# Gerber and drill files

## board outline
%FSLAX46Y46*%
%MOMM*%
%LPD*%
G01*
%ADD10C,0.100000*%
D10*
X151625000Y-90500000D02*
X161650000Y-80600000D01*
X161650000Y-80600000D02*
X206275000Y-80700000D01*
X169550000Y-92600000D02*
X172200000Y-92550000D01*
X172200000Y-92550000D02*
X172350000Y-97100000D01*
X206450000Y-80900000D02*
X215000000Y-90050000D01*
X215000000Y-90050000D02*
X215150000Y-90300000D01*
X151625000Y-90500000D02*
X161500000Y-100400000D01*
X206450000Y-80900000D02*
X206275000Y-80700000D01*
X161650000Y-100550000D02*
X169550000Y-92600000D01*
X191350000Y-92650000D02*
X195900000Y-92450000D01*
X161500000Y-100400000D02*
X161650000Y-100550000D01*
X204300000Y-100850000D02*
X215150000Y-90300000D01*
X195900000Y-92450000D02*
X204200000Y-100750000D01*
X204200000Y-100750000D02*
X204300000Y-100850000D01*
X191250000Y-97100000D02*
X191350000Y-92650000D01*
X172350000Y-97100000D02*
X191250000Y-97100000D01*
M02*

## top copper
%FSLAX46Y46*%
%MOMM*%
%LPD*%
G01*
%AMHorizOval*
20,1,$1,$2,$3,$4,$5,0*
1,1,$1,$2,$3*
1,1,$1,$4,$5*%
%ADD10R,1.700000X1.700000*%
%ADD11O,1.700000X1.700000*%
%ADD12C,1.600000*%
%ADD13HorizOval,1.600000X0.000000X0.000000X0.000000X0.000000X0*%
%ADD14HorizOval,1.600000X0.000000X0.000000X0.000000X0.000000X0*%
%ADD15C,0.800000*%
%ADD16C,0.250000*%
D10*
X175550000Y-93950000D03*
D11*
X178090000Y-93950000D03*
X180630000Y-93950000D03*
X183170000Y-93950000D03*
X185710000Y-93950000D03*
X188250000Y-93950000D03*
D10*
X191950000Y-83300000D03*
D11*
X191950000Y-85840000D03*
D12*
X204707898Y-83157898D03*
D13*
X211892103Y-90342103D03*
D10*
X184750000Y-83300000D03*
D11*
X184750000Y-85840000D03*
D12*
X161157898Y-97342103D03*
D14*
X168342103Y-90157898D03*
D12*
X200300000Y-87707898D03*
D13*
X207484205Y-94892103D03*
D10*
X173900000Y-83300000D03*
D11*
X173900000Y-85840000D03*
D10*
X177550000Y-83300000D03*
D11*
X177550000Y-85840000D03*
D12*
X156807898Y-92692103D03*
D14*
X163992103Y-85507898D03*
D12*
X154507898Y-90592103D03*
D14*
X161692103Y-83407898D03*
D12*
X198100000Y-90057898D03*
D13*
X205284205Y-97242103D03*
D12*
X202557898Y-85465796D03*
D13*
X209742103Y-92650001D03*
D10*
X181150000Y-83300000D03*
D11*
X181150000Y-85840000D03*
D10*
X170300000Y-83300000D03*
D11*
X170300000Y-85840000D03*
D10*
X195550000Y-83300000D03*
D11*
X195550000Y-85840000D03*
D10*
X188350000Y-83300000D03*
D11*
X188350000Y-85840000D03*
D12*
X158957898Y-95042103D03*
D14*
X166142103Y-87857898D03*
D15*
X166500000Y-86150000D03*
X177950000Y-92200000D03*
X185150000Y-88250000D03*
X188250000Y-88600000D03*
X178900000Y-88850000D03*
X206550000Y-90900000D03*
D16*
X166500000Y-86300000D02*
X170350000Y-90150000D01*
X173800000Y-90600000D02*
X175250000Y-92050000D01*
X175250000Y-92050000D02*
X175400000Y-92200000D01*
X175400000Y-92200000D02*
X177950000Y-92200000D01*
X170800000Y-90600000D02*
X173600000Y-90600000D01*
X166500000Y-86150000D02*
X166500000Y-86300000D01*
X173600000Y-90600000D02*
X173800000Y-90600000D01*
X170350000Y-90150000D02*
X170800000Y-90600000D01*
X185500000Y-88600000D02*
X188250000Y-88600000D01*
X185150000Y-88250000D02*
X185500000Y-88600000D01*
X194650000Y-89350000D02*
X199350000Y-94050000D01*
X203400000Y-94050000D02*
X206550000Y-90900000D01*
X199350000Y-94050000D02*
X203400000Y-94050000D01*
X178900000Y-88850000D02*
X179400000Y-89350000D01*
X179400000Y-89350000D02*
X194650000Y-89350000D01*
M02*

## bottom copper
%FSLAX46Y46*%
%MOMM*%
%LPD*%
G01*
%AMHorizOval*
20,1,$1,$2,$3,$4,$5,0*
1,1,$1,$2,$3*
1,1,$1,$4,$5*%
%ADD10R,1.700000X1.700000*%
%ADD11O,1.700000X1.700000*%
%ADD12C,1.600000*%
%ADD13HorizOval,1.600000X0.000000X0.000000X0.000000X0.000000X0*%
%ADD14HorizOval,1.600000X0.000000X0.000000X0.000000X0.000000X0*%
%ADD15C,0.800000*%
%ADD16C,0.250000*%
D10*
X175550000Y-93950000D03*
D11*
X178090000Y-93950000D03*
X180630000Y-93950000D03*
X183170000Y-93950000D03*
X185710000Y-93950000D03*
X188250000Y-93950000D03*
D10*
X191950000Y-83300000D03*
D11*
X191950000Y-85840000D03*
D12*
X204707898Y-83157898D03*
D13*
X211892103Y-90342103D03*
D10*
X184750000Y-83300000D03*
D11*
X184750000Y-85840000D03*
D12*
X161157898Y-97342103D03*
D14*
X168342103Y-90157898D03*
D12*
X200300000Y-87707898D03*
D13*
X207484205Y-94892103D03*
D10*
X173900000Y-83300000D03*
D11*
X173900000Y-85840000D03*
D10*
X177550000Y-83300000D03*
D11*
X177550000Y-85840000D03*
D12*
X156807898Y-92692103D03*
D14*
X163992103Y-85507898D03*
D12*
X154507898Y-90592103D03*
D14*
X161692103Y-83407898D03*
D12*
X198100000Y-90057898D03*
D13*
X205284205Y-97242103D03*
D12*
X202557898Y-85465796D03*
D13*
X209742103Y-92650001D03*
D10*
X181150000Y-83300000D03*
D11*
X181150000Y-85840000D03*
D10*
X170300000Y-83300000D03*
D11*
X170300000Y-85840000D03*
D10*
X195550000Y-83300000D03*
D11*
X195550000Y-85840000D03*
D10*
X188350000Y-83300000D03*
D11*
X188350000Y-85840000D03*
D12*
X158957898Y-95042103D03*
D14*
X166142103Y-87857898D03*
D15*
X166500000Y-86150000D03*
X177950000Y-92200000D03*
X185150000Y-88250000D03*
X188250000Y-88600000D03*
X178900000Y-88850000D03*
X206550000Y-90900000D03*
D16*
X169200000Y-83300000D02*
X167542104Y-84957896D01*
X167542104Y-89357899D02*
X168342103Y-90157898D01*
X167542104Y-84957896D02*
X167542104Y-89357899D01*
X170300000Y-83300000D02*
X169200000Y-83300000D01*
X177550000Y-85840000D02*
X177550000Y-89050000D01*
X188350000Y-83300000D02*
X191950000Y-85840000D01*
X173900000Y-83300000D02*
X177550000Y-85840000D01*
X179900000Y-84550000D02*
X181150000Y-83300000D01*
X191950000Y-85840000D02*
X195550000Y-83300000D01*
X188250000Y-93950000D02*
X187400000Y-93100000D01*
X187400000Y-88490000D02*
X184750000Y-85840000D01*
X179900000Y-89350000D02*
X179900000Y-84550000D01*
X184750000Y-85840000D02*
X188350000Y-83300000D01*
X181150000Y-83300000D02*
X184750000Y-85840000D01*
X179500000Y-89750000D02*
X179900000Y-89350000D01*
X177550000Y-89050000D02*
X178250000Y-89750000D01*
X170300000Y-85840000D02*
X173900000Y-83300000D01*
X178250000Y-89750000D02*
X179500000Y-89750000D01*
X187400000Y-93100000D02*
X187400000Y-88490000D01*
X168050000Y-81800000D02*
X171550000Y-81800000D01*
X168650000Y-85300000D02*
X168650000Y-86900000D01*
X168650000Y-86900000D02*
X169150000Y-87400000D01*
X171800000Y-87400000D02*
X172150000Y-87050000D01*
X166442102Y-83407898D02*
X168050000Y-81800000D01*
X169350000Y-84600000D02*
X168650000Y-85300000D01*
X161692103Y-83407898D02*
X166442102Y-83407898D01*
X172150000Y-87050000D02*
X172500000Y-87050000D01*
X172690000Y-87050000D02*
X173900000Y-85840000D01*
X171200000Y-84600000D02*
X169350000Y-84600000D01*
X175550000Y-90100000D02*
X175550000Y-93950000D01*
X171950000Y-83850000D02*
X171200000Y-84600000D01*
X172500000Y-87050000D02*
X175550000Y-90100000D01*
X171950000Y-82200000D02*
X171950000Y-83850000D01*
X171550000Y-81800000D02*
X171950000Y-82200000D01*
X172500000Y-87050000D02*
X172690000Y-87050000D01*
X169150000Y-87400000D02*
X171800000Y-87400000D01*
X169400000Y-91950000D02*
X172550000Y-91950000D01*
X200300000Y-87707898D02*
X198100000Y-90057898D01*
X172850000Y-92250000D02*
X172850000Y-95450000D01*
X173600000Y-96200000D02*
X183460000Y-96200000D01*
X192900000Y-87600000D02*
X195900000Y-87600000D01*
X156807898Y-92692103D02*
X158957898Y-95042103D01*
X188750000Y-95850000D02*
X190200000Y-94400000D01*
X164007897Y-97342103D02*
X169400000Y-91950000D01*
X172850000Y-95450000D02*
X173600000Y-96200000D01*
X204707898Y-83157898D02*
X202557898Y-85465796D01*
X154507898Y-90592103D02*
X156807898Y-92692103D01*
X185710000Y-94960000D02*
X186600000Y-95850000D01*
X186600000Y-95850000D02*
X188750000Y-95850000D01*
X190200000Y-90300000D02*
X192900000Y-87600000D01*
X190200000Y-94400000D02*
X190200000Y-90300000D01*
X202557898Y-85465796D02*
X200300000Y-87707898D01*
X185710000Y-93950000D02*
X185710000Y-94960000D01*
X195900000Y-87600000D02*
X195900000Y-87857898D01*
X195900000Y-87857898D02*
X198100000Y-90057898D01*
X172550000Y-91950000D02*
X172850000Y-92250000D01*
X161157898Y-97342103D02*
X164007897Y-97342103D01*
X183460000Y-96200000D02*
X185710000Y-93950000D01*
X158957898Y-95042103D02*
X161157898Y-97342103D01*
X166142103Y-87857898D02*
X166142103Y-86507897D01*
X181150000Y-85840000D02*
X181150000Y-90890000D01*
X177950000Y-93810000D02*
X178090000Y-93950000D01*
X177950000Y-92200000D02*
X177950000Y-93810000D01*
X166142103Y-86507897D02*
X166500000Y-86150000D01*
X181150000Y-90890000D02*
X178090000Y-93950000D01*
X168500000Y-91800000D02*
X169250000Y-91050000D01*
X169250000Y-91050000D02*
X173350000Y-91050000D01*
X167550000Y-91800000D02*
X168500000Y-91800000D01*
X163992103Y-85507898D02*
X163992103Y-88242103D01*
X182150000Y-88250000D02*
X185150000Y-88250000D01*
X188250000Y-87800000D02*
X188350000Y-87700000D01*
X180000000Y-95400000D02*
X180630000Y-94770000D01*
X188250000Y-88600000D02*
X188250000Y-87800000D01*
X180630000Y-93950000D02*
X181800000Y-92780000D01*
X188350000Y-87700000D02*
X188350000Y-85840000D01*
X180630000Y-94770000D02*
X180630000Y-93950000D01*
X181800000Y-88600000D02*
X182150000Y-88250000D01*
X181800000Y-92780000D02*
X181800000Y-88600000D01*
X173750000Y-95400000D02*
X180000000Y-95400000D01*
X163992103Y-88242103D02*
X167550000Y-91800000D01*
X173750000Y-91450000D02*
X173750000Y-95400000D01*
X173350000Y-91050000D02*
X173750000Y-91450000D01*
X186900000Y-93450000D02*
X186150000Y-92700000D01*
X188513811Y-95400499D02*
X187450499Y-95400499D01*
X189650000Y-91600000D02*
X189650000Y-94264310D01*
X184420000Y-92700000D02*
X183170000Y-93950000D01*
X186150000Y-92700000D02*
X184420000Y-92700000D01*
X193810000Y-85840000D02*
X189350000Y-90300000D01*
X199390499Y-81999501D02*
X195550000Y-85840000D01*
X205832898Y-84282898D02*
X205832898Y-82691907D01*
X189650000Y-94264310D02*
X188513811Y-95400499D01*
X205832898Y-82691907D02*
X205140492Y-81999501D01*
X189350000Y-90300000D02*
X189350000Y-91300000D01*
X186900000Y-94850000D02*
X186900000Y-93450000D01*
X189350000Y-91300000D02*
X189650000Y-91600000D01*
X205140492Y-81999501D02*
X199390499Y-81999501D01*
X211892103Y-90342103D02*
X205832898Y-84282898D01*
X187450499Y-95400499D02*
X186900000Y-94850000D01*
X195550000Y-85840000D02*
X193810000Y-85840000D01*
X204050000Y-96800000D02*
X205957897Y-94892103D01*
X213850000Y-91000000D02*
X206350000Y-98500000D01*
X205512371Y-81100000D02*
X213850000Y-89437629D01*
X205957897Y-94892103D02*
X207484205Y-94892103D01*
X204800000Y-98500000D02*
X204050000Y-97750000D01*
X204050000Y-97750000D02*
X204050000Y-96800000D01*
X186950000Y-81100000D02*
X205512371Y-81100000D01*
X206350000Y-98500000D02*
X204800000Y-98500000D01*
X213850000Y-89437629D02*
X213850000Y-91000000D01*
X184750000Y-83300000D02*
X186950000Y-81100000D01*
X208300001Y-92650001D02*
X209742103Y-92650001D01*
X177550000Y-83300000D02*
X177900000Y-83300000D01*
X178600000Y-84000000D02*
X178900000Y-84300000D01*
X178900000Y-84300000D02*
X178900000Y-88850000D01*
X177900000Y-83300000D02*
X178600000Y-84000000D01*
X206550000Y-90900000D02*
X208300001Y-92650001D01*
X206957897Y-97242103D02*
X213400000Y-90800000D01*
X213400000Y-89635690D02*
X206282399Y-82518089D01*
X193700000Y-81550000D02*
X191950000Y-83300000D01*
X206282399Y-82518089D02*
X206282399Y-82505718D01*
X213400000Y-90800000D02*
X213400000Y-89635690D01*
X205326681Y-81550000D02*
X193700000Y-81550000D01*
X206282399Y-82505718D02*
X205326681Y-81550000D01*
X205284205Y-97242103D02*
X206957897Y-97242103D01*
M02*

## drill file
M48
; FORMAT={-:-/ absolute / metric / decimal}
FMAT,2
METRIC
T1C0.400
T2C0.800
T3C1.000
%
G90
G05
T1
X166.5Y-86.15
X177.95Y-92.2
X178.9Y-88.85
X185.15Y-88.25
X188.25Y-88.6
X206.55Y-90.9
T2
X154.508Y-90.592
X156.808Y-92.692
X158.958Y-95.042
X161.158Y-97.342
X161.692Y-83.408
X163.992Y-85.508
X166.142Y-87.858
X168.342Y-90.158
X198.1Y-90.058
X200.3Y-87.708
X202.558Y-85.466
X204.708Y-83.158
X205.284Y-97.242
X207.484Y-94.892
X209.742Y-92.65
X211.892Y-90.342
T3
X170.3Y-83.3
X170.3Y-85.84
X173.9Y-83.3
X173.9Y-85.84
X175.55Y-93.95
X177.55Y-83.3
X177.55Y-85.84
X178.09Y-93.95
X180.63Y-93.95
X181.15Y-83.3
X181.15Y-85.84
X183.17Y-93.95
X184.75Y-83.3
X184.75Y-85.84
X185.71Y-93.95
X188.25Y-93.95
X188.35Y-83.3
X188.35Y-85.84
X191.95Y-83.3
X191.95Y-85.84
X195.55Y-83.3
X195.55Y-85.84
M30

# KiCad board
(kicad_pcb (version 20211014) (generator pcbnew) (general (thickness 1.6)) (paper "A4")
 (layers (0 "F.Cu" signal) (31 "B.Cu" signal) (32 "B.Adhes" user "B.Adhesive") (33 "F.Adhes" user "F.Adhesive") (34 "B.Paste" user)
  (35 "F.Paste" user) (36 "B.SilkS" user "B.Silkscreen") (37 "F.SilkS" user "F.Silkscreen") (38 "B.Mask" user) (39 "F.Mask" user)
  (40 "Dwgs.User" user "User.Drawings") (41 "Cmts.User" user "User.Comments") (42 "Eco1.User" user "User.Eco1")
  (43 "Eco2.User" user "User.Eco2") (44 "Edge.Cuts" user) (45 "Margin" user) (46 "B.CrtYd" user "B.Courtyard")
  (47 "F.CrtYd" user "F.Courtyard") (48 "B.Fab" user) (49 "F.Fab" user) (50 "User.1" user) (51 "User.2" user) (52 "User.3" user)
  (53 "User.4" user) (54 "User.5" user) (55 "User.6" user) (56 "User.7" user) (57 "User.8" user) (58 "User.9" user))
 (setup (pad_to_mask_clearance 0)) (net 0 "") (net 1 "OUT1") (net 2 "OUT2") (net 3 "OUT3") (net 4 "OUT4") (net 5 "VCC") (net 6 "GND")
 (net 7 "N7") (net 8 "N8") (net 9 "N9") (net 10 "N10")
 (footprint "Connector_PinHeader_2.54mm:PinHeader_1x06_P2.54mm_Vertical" (layer "F.Cu") (at 175.55 93.95 90)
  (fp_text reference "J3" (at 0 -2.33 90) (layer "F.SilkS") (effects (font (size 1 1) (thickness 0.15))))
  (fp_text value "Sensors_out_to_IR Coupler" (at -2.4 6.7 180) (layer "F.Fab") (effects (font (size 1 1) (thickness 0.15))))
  (pad "1" thru_hole rect (at 0 0 90) (size 1.7 1.7) (drill 1) (layers *.Cu *.Mask) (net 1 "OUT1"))
  (pad "2" thru_hole oval (at 0 2.54 90) (size 1.7 1.7) (drill 1) (layers *.Cu *.Mask) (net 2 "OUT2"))
  (pad "3" thru_hole oval (at 0 5.08 90) (size 1.7 1.7) (drill 1) (layers *.Cu *.Mask) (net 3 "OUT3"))
  (pad "4" thru_hole oval (at 0 7.62 90) (size 1.7 1.7) (drill 1) (layers *.Cu *.Mask) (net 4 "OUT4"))
  (pad "5" thru_hole oval (at 0 10.16 90) (size 1.7 1.7) (drill 1) (layers *.Cu *.Mask) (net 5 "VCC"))
  (pad "6" thru_hole oval (at 0 12.7 90) (size 1.7 1.7) (drill 1) (layers *.Cu *.Mask) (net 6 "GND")))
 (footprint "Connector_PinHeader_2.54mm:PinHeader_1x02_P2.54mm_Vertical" (layer "F.Cu") (at 191.95 83.3)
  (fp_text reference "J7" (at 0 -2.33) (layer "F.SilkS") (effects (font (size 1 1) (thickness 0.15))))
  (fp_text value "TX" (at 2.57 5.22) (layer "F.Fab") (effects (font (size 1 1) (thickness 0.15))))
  (pad "1" thru_hole rect (at 0 0) (size 1.7 1.7) (drill 1) (layers *.Cu *.Mask) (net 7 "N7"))
  (pad "2" thru_hole oval (at 0 2.54) (size 1.7 1.7) (drill 1) (layers *.Cu *.Mask) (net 6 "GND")))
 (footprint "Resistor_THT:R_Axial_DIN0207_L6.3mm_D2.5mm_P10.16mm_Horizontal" (layer "F.Cu") (at 204.707898 83.157898 -45)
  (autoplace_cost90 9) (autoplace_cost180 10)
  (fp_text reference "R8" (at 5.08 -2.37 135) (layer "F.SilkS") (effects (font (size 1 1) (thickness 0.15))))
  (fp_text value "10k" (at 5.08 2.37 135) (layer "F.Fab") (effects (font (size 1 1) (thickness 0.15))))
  (pad "1" thru_hole circle (at 0 0 315) (size 1.6 1.6) (drill 0.8) (layers *.Cu *.Mask) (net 5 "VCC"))
  (pad "2" thru_hole oval (at 10.16 0 315) (size 1.6 1.6) (drill 0.8) (layers *.Cu *.Mask) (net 4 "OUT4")))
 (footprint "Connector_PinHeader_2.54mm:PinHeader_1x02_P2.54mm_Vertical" (layer "F.Cu") (at 184.75 83.3)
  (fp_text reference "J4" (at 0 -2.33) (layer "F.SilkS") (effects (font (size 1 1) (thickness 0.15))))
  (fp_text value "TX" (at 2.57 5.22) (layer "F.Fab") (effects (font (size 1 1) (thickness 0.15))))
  (pad "1" thru_hole rect (at 0 0) (size 1.7 1.7) (drill 1) (layers *.Cu *.Mask) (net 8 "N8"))
  (pad "2" thru_hole oval (at 0 2.54) (size 1.7 1.7) (drill 1) (layers *.Cu *.Mask) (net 6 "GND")))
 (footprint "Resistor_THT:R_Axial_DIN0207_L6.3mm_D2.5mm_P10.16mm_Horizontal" (layer "F.Cu") (at 161.157898 97.342103 45)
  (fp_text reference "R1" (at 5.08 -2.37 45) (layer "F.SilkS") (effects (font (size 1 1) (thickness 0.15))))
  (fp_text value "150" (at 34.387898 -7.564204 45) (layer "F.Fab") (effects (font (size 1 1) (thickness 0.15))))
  (pad "1" thru_hole circle (at 0 0 45) (size 1.6 1.6) (drill 0.8) (layers *.Cu *.Mask) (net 5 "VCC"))
  (pad "2" thru_hole oval (at 10.16 0 45) (size 1.6 1.6) (drill 0.8) (layers *.Cu *.Mask) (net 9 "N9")))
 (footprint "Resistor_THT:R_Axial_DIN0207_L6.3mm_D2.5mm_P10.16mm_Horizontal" (layer "F.Cu") (at 200.3 87.707898 -45)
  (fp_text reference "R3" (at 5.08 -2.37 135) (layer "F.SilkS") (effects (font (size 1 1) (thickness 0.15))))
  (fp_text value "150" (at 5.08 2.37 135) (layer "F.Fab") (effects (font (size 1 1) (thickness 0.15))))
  (pad "1" thru_hole circle (at 0 0 315) (size 1.6 1.6) (drill 0.8) (layers *.Cu *.Mask) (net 5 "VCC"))
  (pad "2" thru_hole oval (at 10.16 0 315) (size 1.6 1.6) (drill 0.8) (layers *.Cu *.Mask) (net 8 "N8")))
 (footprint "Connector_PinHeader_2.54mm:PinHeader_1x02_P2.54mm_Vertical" (layer "F.Cu") (at 173.9 83.3)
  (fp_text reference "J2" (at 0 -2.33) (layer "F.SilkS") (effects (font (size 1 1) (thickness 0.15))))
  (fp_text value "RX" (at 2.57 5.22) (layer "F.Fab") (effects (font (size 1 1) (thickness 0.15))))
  (pad "1" thru_hole rect (at 0 0) (size 1.7 1.7) (drill 1) (layers *.Cu *.Mask) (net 6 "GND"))
  (pad "2" thru_hole oval (at 0 2.54) (size 1.7 1.7) (drill 1) (layers *.Cu *.Mask) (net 1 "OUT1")))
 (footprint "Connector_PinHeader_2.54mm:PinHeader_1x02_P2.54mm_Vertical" (layer "F.Cu") (at 177.55 83.3)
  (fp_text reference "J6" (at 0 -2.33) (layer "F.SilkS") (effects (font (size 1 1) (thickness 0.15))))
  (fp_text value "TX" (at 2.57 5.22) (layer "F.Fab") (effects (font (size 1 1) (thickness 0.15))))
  (pad "1" thru_hole rect (at 0 0) (size 1.7 1.7) (drill 1) (layers *.Cu *.Mask) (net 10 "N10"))
  (pad "2" thru_hole oval (at 0 2.54) (size 1.7 1.7) (drill 1) (layers *.Cu *.Mask) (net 6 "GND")))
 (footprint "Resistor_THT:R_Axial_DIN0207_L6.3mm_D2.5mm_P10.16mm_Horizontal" (layer "F.Cu") (at 156.807898 92.692103 45)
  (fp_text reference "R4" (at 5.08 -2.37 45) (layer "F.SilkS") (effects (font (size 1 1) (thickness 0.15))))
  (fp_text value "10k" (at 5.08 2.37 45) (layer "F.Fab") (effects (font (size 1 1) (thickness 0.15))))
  (pad "1" thru_hole circle (at 0 0 45) (size 1.6 1.6) (drill 0.8) (layers *.Cu *.Mask) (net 5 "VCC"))
  (pad "2" thru_hole oval (at 10.16 0 45) (size 1.6 1.6) (drill 0.8) (layers *.Cu *.Mask) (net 3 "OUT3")))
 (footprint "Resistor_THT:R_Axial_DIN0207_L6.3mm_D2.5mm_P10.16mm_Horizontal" (layer "F.Cu") (at 154.507898 90.592103 45)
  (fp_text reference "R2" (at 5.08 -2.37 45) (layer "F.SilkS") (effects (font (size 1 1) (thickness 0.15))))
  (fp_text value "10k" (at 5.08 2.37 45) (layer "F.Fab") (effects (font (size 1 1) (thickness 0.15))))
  (pad "1" thru_hole circle (at 0 0 45) (size 1.6 1.6) (drill 0.8) (layers *.Cu *.Mask) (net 5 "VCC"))
  (pad "2" thru_hole oval (at 10.16 0 45) (size 1.6 1.6) (drill 0.8) (layers *.Cu *.Mask) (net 1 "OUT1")))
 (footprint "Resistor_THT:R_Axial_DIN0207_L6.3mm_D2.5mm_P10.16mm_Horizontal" (layer "F.Cu") (at 198.1 90.057898 -45)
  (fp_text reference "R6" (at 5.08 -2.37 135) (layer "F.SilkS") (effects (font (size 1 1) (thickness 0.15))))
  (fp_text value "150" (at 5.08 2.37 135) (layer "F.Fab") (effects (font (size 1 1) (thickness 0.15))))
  (pad "1" thru_hole circle (at 0 0 315) (size 1.6 1.6) (drill 0.8) (layers *.Cu *.Mask) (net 5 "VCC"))
  (pad "2" thru_hole oval (at 10.16 0 315) (size 1.6 1.6) (drill 0.8) (layers *.Cu *.Mask) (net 7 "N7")))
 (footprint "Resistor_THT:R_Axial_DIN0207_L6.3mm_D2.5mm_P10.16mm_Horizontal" (layer "F.Cu") (at 202.557898 85.465796 -45)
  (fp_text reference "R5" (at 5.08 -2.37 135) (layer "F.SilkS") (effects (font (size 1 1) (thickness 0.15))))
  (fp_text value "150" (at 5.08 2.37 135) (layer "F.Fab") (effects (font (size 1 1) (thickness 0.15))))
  (pad "1" thru_hole circle (at 0 0 315) (size 1.6 1.6) (drill 0.8) (layers *.Cu *.Mask) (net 5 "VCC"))
  (pad "2" thru_hole oval (at 10.16 0 315) (size 1.6 1.6) (drill 0.8) (layers *.Cu *.Mask) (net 10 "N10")))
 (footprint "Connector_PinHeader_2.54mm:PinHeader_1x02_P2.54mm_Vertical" (layer "F.Cu") (at 181.15 83.3)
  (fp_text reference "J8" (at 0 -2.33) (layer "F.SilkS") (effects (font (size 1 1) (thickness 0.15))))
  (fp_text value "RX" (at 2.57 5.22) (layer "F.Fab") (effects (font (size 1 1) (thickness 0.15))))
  (pad "1" thru_hole rect (at 0 0) (size 1.7 1.7) (drill 1) (layers *.Cu *.Mask) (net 6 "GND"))
  (pad "2" thru_hole oval (at 0 2.54) (size 1.7 1.7) (drill 1) (layers *.Cu *.Mask) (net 2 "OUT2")))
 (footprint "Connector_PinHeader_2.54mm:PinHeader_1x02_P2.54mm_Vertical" (layer "F.Cu") (at 170.3 83.3)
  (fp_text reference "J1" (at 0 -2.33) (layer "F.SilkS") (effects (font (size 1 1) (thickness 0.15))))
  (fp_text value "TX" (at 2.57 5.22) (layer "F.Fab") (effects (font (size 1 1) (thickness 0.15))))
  (pad "1" thru_hole rect (at 0 0) (size 1.7 1.7) (drill 1) (layers *.Cu *.Mask) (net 9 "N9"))
  (pad "2" thru_hole oval (at 0 2.54) (size 1.7 1.7) (drill 1) (layers *.Cu *.Mask) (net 6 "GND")))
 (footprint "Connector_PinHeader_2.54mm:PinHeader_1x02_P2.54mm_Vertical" (layer "F.Cu") (at 195.55 83.3)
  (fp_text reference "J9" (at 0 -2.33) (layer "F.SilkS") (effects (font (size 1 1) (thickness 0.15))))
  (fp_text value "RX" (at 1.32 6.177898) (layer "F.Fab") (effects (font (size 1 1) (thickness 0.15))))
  (pad "1" thru_hole rect (at 0 0) (size 1.7 1.7) (drill 1) (layers *.Cu *.Mask) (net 6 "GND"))
  (pad "2" thru_hole oval (at 0 2.54) (size 1.7 1.7) (drill 1) (layers *.Cu *.Mask) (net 4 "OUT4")))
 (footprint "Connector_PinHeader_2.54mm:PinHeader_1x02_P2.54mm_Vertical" (layer "F.Cu") (at 188.35 83.3)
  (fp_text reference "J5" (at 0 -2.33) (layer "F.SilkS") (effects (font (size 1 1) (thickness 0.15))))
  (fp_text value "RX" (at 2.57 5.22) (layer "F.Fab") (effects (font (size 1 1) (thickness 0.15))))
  (pad "1" thru_hole rect (at 0 0) (size 1.7 1.7) (drill 1) (layers *.Cu *.Mask) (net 6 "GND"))
  (pad "2" thru_hole oval (at 0 2.54) (size 1.7 1.7) (drill 1) (layers *.Cu *.Mask) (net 3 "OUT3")))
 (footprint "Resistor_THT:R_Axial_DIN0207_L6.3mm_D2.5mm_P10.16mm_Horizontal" (layer "F.Cu") (at 158.957898 95.042103 45)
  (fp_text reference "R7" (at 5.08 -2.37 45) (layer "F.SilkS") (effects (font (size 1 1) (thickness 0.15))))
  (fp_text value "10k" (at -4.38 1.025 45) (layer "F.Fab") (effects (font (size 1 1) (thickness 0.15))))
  (pad "1" thru_hole circle (at 0 0 45) (size 1.6 1.6) (drill 0.8) (layers *.Cu *.Mask) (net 5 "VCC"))
  (pad "2" thru_hole oval (at 10.16 0 45) (size 1.6 1.6) (drill 0.8) (layers *.Cu *.Mask) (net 2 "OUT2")))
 (gr_line (start 151.625 90.5) (end 161.65 80.6) (layer "Edge.Cuts") (width 0.1))
 (gr_line (start 161.65 80.6) (end 206.275 80.7) (layer "Edge.Cuts") (width 0.1))
 (gr_line (start 169.55 92.6) (end 172.2 92.55) (layer "Edge.Cuts") (width 0.1))
 (gr_line (start 172.2 92.55) (end 172.35 97.1) (layer "Edge.Cuts") (width 0.1))
 (gr_line (start 206.45 80.9) (end 215 90.05) (layer "Edge.Cuts") (width 0.1))
 (gr_line (start 215 90.05) (end 215.15 90.3) (layer "Edge.Cuts") (width 0.1))
 (gr_line (start 151.625 90.5) (end 161.5 100.4) (layer "Edge.Cuts") (width 0.1))
 (gr_line (start 206.45 80.9) (end 206.275 80.7) (layer "Edge.Cuts") (width 0.1))
 (gr_line (start 161.65 100.55) (end 169.55 92.6) (layer "Edge.Cuts") (width 0.1))
 (gr_line (start 191.35 92.65) (end 195.9 92.45) (layer "Edge.Cuts") (width 0.1))
 (gr_line (start 161.5 100.4) (end 161.65 100.55) (layer "Edge.Cuts") (width 0.1))
 (gr_line (start 204.3 100.85) (end 215.15 90.3) (layer "Edge.Cuts") (width 0.1))
 (gr_line (start 195.9 92.45) (end 204.2 100.75) (layer "Edge.Cuts") (width 0.1))
 (gr_line (start 204.2 100.75) (end 204.3 100.85) (layer "Edge.Cuts") (width 0.1))
 (gr_line (start 191.25 97.1) (end 191.35 92.65) (layer "Edge.Cuts") (width 0.1))
 (gr_line (start 172.35 97.1) (end 191.25 97.1) (layer "Edge.Cuts") (width 0.1))
 (segment (start 169.2 83.3) (end 167.542104 84.957896) (width 0.25) (layer "B.Cu") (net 9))
 (segment (start 167.542104 89.357899) (end 168.342103 90.157898) (width 0.25) (layer "B.Cu") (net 9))
 (segment (start 167.542104 84.957896) (end 167.542104 89.357899) (width 0.25) (layer "B.Cu") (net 9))
 (segment (start 170.3 83.3) (end 169.2 83.3) (width 0.25) (layer "B.Cu") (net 9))
 (segment (start 177.55 85.84) (end 177.55 89.05) (width 0.25) (layer "B.Cu") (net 6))
 (segment (start 188.35 83.3) (end 191.95 85.84) (width 0.25) (layer "B.Cu") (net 6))
 (segment (start 173.9 83.3) (end 177.55 85.84) (width 0.25) (layer "B.Cu") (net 6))
 (segment (start 179.9 84.55) (end 181.15 83.3) (width 0.25) (layer "B.Cu") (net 6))
 (segment (start 191.95 85.84) (end 195.55 83.3) (width 0.25) (layer "B.Cu") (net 6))
 (segment (start 188.25 93.95) (end 187.4 93.1) (width 0.25) (layer "B.Cu") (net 6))
 (segment (start 187.4 88.49) (end 184.75 85.84) (width 0.25) (layer "B.Cu") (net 6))
 (segment (start 179.9 89.35) (end 179.9 84.55) (width 0.25) (layer "B.Cu") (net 6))
 (segment (start 184.75 85.84) (end 188.35 83.3) (width 0.25) (layer "B.Cu") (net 6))
 (segment (start 181.15 83.3) (end 184.75 85.84) (width 0.25) (layer "B.Cu") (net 6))
 (segment (start 179.5 89.75) (end 179.9 89.35) (width 0.25) (layer "B.Cu") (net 6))
 (segment (start 177.55 89.05) (end 178.25 89.75) (width 0.25) (layer "B.Cu") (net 6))
 (segment (start 170.3 85.84) (end 173.9 83.3) (width 0.25) (layer "B.Cu") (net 6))
 (segment (start 178.25 89.75) (end 179.5 89.75) (width 0.25) (layer "B.Cu") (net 6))
 (segment (start 187.4 93.1) (end 187.4 88.49) (width 0.25) (layer "B.Cu") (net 6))
 (segment (start 168.05 81.8) (end 171.55 81.8) (width 0.25) (layer "B.Cu") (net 1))
 (segment (start 168.65 85.3) (end 168.65 86.9) (width 0.25) (layer "B.Cu") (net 1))
 (segment (start 168.65 86.9) (end 169.15 87.4) (width 0.25) (layer "B.Cu") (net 1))
 (segment (start 171.8 87.4) (end 172.15 87.05) (width 0.25) (layer "B.Cu") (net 1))
 (segment (start 166.442102 83.407898) (end 168.05 81.8) (width 0.25) (layer "B.Cu") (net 1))
 (segment (start 169.35 84.6) (end 168.65 85.3) (width 0.25) (layer "B.Cu") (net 1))
 (segment (start 161.692103 83.407898) (end 166.442102 83.407898) (width 0.25) (layer "B.Cu") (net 1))
 (segment (start 172.15 87.05) (end 172.5 87.05) (width 0.25) (layer "B.Cu") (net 1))
 (segment (start 172.69 87.05) (end 173.9 85.84) (width 0.25) (layer "B.Cu") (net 1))
 (segment (start 171.2 84.6) (end 169.35 84.6) (width 0.25) (layer "B.Cu") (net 1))
 (segment (start 175.55 90.1) (end 175.55 93.95) (width 0.25) (layer "B.Cu") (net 1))
 (segment (start 171.95 83.85) (end 171.2 84.6) (width 0.25) (layer "B.Cu") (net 1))
 (segment (start 172.5 87.05) (end 175.55 90.1) (width 0.25) (layer "B.Cu") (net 1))
 (segment (start 171.95 82.2) (end 171.95 83.85) (width 0.25) (layer "B.Cu") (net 1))
 (segment (start 171.55 81.8) (end 171.95 82.2) (width 0.25) (layer "B.Cu") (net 1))
 (segment (start 172.5 87.05) (end 172.69 87.05) (width 0.25) (layer "B.Cu") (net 1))
 (segment (start 169.15 87.4) (end 171.8 87.4) (width 0.25) (layer "B.Cu") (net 1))
 (segment (start 169.4 91.95) (end 172.55 91.95) (width 0.25) (layer "B.Cu") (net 5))
 (segment (start 200.3 87.707898) (end 198.1 90.057898) (width 0.25) (layer "B.Cu") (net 5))
 (segment (start 172.85 92.25) (end 172.85 95.45) (width 0.25) (layer "B.Cu") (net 5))
 (segment (start 173.6 96.2) (end 183.46 96.2) (width 0.25) (layer "B.Cu") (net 5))
 (segment (start 192.9 87.6) (end 195.9 87.6) (width 0.25) (layer "B.Cu") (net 5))
 (segment (start 156.807898 92.692103) (end 158.957898 95.042103) (width 0.25) (layer "B.Cu") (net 5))
 (segment (start 188.75 95.85) (end 190.2 94.4) (width 0.25) (layer "B.Cu") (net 5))
 (segment (start 164.007897 97.342103) (end 169.4 91.95) (width 0.25) (layer "B.Cu") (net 5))
 (segment (start 172.85 95.45) (end 173.6 96.2) (width 0.25) (layer "B.Cu") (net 5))
 (segment (start 204.707898 83.157898) (end 202.557898 85.465796) (width 0.25) (layer "B.Cu") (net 5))
 (segment (start 154.507898 90.592103) (end 156.807898 92.692103) (width 0.25) (layer "B.Cu") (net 5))
 (segment (start 185.71 94.96) (end 186.6 95.85) (width 0.25) (layer "B.Cu") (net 5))
 (segment (start 186.6 95.85) (end 188.75 95.85) (width 0.25) (layer "B.Cu") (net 5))
 (segment (start 190.2 90.3) (end 192.9 87.6) (width 0.25) (layer "B.Cu") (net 5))
 (segment (start 190.2 94.4) (end 190.2 90.3) (width 0.25) (layer "B.Cu") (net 5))
 (segment (start 202.557898 85.465796) (end 200.3 87.707898) (width 0.25) (layer "B.Cu") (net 5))
 (segment (start 185.71 93.95) (end 185.71 94.96) (width 0.25) (layer "B.Cu") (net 5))
 (segment (start 195.9 87.6) (end 195.9 87.857898) (width 0.25) (layer "B.Cu") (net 5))
 (segment (start 195.9 87.857898) (end 198.1 90.057898) (width 0.25) (layer "B.Cu") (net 5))
 (segment (start 172.55 91.95) (end 172.85 92.25) (width 0.25) (layer "B.Cu") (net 5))
 (segment (start 161.157898 97.342103) (end 164.007897 97.342103) (width 0.25) (layer "B.Cu") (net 5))
 (segment (start 183.46 96.2) (end 185.71 93.95) (width 0.25) (layer "B.Cu") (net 5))
 (segment (start 158.957898 95.042103) (end 161.157898 97.342103) (width 0.25) (layer "B.Cu") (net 5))
 (segment (start 166.5 86.3) (end 170.35 90.15) (width 0.25) (layer "F.Cu") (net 2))
 (segment (start 173.8 90.6) (end 175.25 92.05) (width 0.25) (layer "F.Cu") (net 2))
 (segment (start 175.25 92.05) (end 175.4 92.2) (width 0.25) (layer "F.Cu") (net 2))
 (segment (start 175.4 92.2) (end 177.95 92.2) (width 0.25) (layer "F.Cu") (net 2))
 (segment (start 170.8 90.6) (end 173.6 90.6) (width 0.25) (layer "F.Cu") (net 2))
 (segment (start 166.5 86.15) (end 166.5 86.3) (width 0.25) (layer "F.Cu") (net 2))
 (segment (start 173.6 90.6) (end 173.8 90.6) (width 0.25) (layer "F.Cu") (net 2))
 (segment (start 170.35 90.15) (end 170.8 90.6) (width 0.25) (layer "F.Cu") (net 2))
 (via (at 166.5 86.15) (size 0.8) (drill 0.4) (layers "F.Cu" "B.Cu") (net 2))
 (via (at 177.95 92.2) (size 0.8) (drill 0.4) (layers "F.Cu" "B.Cu") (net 2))
 (segment (start 166.142103 87.857898) (end 166.142103 86.507897) (width 0.25) (layer "B.Cu") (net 2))
 (segment (start 181.15 85.84) (end 181.15 90.89) (width 0.25) (layer "B.Cu") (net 2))
 (segment (start 177.95 93.81) (end 178.09 93.95) (width 0.25) (layer "B.Cu") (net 2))
 (segment (start 177.95 92.2) (end 177.95 93.81) (width 0.25) (layer "B.Cu") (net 2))
 (segment (start 166.142103 86.507897) (end 166.5 86.15) (width 0.25) (layer "B.Cu") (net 2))
 (segment (start 181.15 90.89) (end 178.09 93.95) (width 0.25) (layer "B.Cu") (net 2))
 (segment (start 185.5 88.6) (end 188.25 88.6) (width 0.25) (layer "F.Cu") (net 3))
 (segment (start 185.15 88.25) (end 185.5 88.6) (width 0.25) (layer "F.Cu") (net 3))
 (via (at 185.15 88.25) (size 0.8) (drill 0.4) (layers "F.Cu" "B.Cu") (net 3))
 (via (at 188.25 88.6) (size 0.8) (drill 0.4) (layers "F.Cu" "B.Cu") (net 3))
 (segment (start 168.5 91.8) (end 169.25 91.05) (width 0.25) (layer "B.Cu") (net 3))
 (segment (start 169.25 91.05) (end 173.35 91.05) (width 0.25) (layer "B.Cu") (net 3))
 (segment (start 167.55 91.8) (end 168.5 91.8) (width 0.25) (layer "B.Cu") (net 3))
 (segment (start 163.992103 85.507898) (end 163.992103 88.242103) (width 0.25) (layer "B.Cu") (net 3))
 (segment (start 182.15 88.25) (end 185.15 88.25) (width 0.25) (layer "B.Cu") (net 3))
 (segment (start 188.25 87.8) (end 188.35 87.7) (width 0.25) (layer "B.Cu") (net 3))
 (segment (start 180 95.4) (end 180.63 94.77) (width 0.25) (layer "B.Cu") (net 3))
 (segment (start 188.25 88.6) (end 188.25 87.8) (width 0.25) (layer "B.Cu") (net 3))
 (segment (start 180.63 93.95) (end 181.8 92.78) (width 0.25) (layer "B.Cu") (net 3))
 (segment (start 188.35 87.7) (end 188.35 85.84) (width 0.25) (layer "B.Cu") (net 3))
 (segment (start 180.63 94.77) (end 180.63 93.95) (width 0.25) (layer "B.Cu") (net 3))
 (segment (start 181.8 88.6) (end 182.15 88.25) (width 0.25) (layer "B.Cu") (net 3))
 (segment (start 181.8 92.78) (end 181.8 88.6) (width 0.25) (layer "B.Cu") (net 3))
 (segment (start 173.75 95.4) (end 180 95.4) (width 0.25) (layer "B.Cu") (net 3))
 (segment (start 163.992103 88.242103) (end 167.55 91.8) (width 0.25) (layer "B.Cu") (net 3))
 (segment (start 173.75 91.45) (end 173.75 95.4) (width 0.25) (layer "B.Cu") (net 3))
 (segment (start 173.35 91.05) (end 173.75 91.45) (width 0.25) (layer "B.Cu") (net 3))
 (segment (start 186.9 93.45) (end 186.15 92.7) (width 0.25) (layer "B.Cu") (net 4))
 (segment (start 188.513811 95.400499) (end 187.450499 95.400499) (width 0.25) (layer "B.Cu") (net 4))
 (segment (start 189.65 91.6) (end 189.65 94.26431) (width 0.25) (layer "B.Cu") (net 4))
 (segment (start 184.42 92.7) (end 183.17 93.95) (width 0.25) (layer "B.Cu") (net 4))
 (segment (start 186.15 92.7) (end 184.42 92.7) (width 0.25) (layer "B.Cu") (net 4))
 (segment (start 193.81 85.84) (end 189.35 90.3) (width 0.25) (layer "B.Cu") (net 4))
 (segment (start 199.390499 81.999501) (end 195.55 85.84) (width 0.25) (layer "B.Cu") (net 4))
 (segment (start 205.832898 84.282898) (end 205.832898 82.691907) (width 0.25) (layer "B.Cu") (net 4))
 (segment (start 189.65 94.26431) (end 188.513811 95.400499) (width 0.25) (layer "B.Cu") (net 4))
 (segment (start 205.832898 82.691907) (end 205.140492 81.999501) (width 0.25) (layer "B.Cu") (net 4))
 (segment (start 189.35 90.3) (end 189.35 91.3) (width 0.25) (layer "B.Cu") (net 4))
 (segment (start 186.9 94.85) (end 186.9 93.45) (width 0.25) (layer "B.Cu") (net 4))
 (segment (start 189.35 91.3) (end 189.65 91.6) (width 0.25) (layer "B.Cu") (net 4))
 (segment (start 205.140492 81.999501) (end 199.390499 81.999501) (width 0.25) (layer "B.Cu") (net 4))
 (segment (start 211.892103 90.342103) (end 205.832898 84.282898) (width 0.25) (layer "B.Cu") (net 4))
 (segment (start 187.450499 95.400499) (end 186.9 94.85) (width 0.25) (layer "B.Cu") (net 4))
 (segment (start 195.55 85.84) (end 193.81 85.84) (width 0.25) (layer "B.Cu") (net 4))
 (segment (start 204.05 96.8) (end 205.957897 94.892103) (width 0.25) (layer "B.Cu") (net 8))
 (segment (start 213.85 91) (end 206.35 98.5) (width 0.25) (layer "B.Cu") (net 8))
 (segment (start 205.512371 81.1) (end 213.85 89.437629) (width 0.25) (layer "B.Cu") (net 8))
 (segment (start 205.957897 94.892103) (end 207.484205 94.892103) (width 0.25) (layer "B.Cu") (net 8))
 (segment (start 204.8 98.5) (end 204.05 97.75) (width 0.25) (layer "B.Cu") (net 8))
 (segment (start 204.05 97.75) (end 204.05 96.8) (width 0.25) (layer "B.Cu") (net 8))
 (segment (start 186.95 81.1) (end 205.512371 81.1) (width 0.25) (layer "B.Cu") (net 8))
 (segment (start 206.35 98.5) (end 204.8 98.5) (width 0.25) (layer "B.Cu") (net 8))
 (segment (start 213.85 89.437629) (end 213.85 91) (width 0.25) (layer "B.Cu") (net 8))
 (segment (start 184.75 83.3) (end 186.95 81.1) (width 0.25) (layer "B.Cu") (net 8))
 (segment (start 194.65 89.35) (end 199.35 94.05) (width 0.25) (layer "F.Cu") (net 10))
 (segment (start 203.4 94.05) (end 206.55 90.9) (width 0.25) (layer "F.Cu") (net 10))
 (segment (start 199.35 94.05) (end 203.4 94.05) (width 0.25) (layer "F.Cu") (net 10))
 (segment (start 178.9 88.85) (end 179.4 89.35) (width 0.25) (layer "F.Cu") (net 10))
 (segment (start 179.4 89.35) (end 194.65 89.35) (width 0.25) (layer "F.Cu") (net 10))
 (via (at 178.9 88.85) (size 0.8) (drill 0.4) (layers "F.Cu" "B.Cu") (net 10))
 (via (at 206.55 90.9) (size 0.8) (drill 0.4) (layers "F.Cu" "B.Cu") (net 10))
 (segment (start 208.300001 92.650001) (end 209.742103 92.650001) (width 0.25) (layer "B.Cu") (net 10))
 (segment (start 177.55 83.3) (end 177.9 83.3) (width 0.25) (layer "B.Cu") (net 10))
 (segment (start 178.6 84) (end 178.9 84.3) (width 0.25) (layer "B.Cu") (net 10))
 (segment (start 178.9 84.3) (end 178.9 88.85) (width 0.25) (layer "B.Cu") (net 10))
 (segment (start 177.9 83.3) (end 178.6 84) (width 0.25) (layer "B.Cu") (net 10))
 (segment (start 206.55 90.9) (end 208.300001 92.650001) (width 0.25) (layer "B.Cu") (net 10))
 (segment (start 206.957897 97.242103) (end 213.4 90.8) (width 0.25) (layer "B.Cu") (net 7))
 (segment (start 213.4 89.63569) (end 206.282399 82.518089) (width 0.25) (layer "B.Cu") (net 7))
 (segment (start 193.7 81.55) (end 191.95 83.3) (width 0.25) (layer "B.Cu") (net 7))
 (segment (start 206.282399 82.518089) (end 206.282399 82.505718) (width 0.25) (layer "B.Cu") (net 7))
 (segment (start 213.4 90.8) (end 213.4 89.63569) (width 0.25) (layer "B.Cu") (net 7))
 (segment (start 205.326681 81.55) (end 193.7 81.55) (width 0.25) (layer "B.Cu") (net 7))
 (segment (start 206.282399 82.505718) (end 205.326681 81.55) (width 0.25) (layer "B.Cu") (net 7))
 (segment (start 205.284205 97.242103) (end 206.957897 97.242103) (width 0.25) (layer "B.Cu") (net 7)))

